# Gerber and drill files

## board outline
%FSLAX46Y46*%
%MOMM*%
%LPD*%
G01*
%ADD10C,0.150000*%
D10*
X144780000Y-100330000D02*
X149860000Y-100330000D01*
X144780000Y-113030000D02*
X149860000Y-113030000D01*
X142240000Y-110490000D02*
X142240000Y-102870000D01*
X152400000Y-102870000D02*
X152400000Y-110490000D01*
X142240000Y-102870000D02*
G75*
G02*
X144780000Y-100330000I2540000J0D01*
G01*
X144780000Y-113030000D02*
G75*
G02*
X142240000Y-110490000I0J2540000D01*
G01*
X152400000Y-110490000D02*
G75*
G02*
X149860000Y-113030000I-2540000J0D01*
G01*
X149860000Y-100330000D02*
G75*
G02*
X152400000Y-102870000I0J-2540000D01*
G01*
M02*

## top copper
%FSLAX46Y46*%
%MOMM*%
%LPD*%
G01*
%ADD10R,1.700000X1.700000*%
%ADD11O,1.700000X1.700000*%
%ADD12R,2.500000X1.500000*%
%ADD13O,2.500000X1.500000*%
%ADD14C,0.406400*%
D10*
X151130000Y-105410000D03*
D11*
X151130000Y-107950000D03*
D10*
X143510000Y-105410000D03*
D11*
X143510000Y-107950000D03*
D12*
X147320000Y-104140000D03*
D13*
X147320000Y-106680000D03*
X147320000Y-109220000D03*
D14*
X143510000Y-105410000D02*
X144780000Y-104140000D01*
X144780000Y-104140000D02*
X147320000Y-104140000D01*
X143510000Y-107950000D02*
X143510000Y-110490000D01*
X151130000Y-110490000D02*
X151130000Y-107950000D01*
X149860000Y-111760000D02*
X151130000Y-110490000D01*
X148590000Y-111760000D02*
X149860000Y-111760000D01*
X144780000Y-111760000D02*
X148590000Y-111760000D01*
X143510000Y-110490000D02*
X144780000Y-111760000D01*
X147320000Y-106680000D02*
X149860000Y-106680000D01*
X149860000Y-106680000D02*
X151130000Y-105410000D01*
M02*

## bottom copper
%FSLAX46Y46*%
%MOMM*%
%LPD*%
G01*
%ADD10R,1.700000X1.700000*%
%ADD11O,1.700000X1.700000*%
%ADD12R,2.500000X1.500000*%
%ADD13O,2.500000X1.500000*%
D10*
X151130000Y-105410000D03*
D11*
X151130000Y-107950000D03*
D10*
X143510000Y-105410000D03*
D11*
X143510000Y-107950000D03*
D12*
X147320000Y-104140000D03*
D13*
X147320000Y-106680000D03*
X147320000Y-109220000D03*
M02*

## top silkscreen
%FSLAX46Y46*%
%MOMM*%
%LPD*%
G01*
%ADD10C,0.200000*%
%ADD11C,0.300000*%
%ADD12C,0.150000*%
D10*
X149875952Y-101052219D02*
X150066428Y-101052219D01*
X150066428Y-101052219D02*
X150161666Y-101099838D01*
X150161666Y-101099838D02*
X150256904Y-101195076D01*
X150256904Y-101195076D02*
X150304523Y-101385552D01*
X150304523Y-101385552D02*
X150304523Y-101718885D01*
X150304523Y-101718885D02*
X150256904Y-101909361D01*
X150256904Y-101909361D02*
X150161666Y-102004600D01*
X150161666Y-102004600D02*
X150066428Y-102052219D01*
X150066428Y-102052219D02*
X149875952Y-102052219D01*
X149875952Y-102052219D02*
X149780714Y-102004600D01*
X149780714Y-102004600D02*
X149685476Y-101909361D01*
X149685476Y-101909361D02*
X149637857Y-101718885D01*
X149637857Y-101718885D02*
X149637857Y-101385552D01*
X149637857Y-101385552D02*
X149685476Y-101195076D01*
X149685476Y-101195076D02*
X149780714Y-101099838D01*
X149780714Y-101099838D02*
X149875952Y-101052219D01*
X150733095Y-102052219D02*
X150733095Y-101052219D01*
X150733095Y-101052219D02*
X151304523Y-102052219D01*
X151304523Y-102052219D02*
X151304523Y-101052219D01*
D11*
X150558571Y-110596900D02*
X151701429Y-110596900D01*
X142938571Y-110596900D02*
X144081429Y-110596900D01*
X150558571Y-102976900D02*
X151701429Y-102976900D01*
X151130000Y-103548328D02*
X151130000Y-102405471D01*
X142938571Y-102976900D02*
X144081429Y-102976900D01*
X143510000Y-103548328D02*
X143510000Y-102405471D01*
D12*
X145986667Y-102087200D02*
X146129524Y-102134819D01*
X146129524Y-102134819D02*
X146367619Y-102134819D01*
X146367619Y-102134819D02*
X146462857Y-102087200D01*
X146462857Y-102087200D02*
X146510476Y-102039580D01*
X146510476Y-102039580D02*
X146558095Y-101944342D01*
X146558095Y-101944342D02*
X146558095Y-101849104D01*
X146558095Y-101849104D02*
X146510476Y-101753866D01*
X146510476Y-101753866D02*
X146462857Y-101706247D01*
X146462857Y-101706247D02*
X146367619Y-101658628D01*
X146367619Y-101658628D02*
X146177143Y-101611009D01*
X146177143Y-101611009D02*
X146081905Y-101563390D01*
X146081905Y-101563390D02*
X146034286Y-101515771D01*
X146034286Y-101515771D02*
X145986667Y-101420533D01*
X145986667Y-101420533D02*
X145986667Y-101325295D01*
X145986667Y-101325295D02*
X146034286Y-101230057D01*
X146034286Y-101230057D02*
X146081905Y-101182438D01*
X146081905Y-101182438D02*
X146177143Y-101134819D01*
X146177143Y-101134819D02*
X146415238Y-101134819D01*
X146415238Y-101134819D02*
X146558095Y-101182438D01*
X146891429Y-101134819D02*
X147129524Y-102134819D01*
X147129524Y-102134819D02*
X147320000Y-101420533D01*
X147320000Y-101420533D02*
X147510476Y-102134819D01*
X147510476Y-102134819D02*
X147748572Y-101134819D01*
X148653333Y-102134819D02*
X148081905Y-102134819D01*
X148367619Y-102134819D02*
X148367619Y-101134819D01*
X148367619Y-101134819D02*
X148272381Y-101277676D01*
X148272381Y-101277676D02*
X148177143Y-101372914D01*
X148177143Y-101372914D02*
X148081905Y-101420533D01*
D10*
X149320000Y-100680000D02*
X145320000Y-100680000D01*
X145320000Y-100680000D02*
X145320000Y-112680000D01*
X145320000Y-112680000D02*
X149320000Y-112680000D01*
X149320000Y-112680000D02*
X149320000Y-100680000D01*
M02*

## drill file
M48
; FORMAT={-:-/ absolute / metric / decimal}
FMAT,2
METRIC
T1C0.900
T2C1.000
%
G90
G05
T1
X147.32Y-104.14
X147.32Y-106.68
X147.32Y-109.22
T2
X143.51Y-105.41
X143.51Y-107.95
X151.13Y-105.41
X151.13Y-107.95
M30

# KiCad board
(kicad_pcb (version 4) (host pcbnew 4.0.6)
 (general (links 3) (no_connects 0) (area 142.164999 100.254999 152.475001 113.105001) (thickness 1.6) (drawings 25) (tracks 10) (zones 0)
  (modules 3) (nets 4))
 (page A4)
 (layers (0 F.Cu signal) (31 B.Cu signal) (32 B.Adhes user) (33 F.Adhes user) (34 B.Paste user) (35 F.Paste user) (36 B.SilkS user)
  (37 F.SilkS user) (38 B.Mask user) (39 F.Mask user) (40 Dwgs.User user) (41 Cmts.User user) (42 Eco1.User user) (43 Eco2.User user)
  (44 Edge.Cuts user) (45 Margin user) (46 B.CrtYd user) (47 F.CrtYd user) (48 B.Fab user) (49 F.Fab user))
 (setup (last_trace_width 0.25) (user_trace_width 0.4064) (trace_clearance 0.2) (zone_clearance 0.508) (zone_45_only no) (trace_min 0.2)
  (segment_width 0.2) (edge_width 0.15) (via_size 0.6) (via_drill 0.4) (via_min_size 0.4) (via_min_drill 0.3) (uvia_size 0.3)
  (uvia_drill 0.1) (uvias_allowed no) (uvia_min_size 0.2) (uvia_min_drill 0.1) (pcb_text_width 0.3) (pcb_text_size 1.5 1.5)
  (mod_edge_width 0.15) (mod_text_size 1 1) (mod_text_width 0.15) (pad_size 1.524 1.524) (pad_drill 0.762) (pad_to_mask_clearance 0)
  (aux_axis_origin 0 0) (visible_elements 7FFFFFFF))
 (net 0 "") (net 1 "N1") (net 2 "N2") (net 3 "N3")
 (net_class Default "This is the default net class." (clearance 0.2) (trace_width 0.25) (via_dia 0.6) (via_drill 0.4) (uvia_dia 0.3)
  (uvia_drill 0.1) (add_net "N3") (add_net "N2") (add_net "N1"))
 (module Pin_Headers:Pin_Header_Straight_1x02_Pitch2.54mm (layer F.Cu) (at 151.13 105.41)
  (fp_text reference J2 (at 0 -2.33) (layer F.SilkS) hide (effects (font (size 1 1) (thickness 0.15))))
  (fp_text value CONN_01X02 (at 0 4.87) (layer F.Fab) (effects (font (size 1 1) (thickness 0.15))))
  (pad 1 thru_hole rect (at 0 0) (size 1.7 1.7) (drill 1) (layers *.Cu *.Mask) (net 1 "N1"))
  (pad 2 thru_hole oval (at 0 2.54) (size 1.7 1.7) (drill 1) (layers *.Cu *.Mask) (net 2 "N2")))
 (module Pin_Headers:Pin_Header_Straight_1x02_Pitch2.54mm (layer F.Cu) (at 143.51 105.41)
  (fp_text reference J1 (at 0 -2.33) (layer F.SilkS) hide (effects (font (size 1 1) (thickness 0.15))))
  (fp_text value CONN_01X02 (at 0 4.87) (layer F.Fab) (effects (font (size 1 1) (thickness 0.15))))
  (pad 1 thru_hole rect (at 0 0) (size 1.7 1.7) (drill 1) (layers *.Cu *.Mask) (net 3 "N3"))
  (pad 2 thru_hole oval (at 0 2.54) (size 1.7 1.7) (drill 1) (layers *.Cu *.Mask) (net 2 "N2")))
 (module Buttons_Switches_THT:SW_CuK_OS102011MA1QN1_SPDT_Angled (layer F.Cu) (at 147.32 106.68 270)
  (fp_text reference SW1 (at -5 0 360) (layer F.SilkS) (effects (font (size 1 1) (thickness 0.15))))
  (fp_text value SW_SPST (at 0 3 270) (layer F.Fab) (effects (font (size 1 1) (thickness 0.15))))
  (fp_line (start -6 -2) (end -6 2) (layer F.SilkS) (width 0.2)) (fp_line (start -6 2) (end 6 2) (layer F.SilkS) (width 0.2))
  (fp_line (start 6 2) (end 6 -2) (layer F.SilkS) (width 0.2))
  (fp_line (start 6 -2) (end -6 -2) (layer F.SilkS) (width 0.2))
  (pad 1 thru_hole rect (at -2.54 0 270) (size 1.5 2.5) (drill 0.9) (layers *.Cu *.Mask) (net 3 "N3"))
  (pad 2 thru_hole oval (at 0 0 270) (size 1.5 2.5) (drill 0.9) (layers *.Cu *.Mask) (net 1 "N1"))
  (pad 3 thru_hole oval (at 2.54 0 270) (size 1.5 2.5) (drill 0.9) (layers *.Cu *.Mask)))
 (gr_line (start 144.78 100.33) (end 149.86 100.33) (angle 90) (layer Edge.Cuts) (width 0.15))
 (gr_line (start 144.78 113.03) (end 149.86 113.03) (angle 90) (layer Edge.Cuts) (width 0.15))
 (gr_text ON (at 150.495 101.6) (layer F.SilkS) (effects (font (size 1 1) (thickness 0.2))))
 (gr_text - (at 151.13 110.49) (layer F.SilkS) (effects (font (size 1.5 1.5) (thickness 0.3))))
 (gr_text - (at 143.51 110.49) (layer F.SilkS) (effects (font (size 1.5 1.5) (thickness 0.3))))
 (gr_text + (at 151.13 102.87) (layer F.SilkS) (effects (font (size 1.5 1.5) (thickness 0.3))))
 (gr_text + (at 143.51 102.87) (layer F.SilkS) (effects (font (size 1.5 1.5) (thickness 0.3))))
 (gr_line (start 142.24 110.49) (end 142.24 102.87) (angle 90) (layer Edge.Cuts) (width 0.15))
 (gr_line (start 152.4 102.87) (end 152.4 110.49) (angle 90) (layer Edge.Cuts) (width 0.15))
 (gr_arc (start 144.78 102.87) (end 142.24 102.87) (angle 90) (layer Edge.Cuts) (width 0.15))
 (gr_arc (start 144.78 110.49) (end 144.78 113.03) (angle 90) (layer Edge.Cuts) (width 0.15))
 (gr_arc (start 149.86 110.49) (end 152.4 110.49) (angle 90) (layer Edge.Cuts) (width 0.15))
 (gr_arc (start 149.86 102.87) (end 149.86 100.33) (angle 90) (layer Edge.Cuts) (width 0.15))
 (segment (start 143.51 105.41) (end 144.78 104.14) (width 0.4064) (layer F.Cu) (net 3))
 (segment (start 144.78 104.14) (end 147.32 104.14) (width 0.4064) (layer F.Cu) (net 3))
 (segment (start 143.51 107.95) (end 143.51 110.49) (width 0.4064) (layer F.Cu) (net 2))
 (segment (start 151.13 110.49) (end 151.13 107.95) (width 0.4064) (layer F.Cu) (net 2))
 (segment (start 149.86 111.76) (end 151.13 110.49) (width 0.4064) (layer F.Cu) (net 2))
 (segment (start 148.59 111.76) (end 149.86 111.76) (width 0.4064) (layer F.Cu) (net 2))
 (segment (start 144.78 111.76) (end 148.59 111.76) (width 0.4064) (layer F.Cu) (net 2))
 (segment (start 143.51 110.49) (end 144.78 111.76) (width 0.4064) (layer F.Cu) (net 2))
 (segment (start 147.32 106.68) (end 149.86 106.68) (width 0.4064) (layer F.Cu) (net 1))
 (segment (start 149.86 106.68) (end 151.13 105.41) (width 0.4064) (layer F.Cu) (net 1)))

